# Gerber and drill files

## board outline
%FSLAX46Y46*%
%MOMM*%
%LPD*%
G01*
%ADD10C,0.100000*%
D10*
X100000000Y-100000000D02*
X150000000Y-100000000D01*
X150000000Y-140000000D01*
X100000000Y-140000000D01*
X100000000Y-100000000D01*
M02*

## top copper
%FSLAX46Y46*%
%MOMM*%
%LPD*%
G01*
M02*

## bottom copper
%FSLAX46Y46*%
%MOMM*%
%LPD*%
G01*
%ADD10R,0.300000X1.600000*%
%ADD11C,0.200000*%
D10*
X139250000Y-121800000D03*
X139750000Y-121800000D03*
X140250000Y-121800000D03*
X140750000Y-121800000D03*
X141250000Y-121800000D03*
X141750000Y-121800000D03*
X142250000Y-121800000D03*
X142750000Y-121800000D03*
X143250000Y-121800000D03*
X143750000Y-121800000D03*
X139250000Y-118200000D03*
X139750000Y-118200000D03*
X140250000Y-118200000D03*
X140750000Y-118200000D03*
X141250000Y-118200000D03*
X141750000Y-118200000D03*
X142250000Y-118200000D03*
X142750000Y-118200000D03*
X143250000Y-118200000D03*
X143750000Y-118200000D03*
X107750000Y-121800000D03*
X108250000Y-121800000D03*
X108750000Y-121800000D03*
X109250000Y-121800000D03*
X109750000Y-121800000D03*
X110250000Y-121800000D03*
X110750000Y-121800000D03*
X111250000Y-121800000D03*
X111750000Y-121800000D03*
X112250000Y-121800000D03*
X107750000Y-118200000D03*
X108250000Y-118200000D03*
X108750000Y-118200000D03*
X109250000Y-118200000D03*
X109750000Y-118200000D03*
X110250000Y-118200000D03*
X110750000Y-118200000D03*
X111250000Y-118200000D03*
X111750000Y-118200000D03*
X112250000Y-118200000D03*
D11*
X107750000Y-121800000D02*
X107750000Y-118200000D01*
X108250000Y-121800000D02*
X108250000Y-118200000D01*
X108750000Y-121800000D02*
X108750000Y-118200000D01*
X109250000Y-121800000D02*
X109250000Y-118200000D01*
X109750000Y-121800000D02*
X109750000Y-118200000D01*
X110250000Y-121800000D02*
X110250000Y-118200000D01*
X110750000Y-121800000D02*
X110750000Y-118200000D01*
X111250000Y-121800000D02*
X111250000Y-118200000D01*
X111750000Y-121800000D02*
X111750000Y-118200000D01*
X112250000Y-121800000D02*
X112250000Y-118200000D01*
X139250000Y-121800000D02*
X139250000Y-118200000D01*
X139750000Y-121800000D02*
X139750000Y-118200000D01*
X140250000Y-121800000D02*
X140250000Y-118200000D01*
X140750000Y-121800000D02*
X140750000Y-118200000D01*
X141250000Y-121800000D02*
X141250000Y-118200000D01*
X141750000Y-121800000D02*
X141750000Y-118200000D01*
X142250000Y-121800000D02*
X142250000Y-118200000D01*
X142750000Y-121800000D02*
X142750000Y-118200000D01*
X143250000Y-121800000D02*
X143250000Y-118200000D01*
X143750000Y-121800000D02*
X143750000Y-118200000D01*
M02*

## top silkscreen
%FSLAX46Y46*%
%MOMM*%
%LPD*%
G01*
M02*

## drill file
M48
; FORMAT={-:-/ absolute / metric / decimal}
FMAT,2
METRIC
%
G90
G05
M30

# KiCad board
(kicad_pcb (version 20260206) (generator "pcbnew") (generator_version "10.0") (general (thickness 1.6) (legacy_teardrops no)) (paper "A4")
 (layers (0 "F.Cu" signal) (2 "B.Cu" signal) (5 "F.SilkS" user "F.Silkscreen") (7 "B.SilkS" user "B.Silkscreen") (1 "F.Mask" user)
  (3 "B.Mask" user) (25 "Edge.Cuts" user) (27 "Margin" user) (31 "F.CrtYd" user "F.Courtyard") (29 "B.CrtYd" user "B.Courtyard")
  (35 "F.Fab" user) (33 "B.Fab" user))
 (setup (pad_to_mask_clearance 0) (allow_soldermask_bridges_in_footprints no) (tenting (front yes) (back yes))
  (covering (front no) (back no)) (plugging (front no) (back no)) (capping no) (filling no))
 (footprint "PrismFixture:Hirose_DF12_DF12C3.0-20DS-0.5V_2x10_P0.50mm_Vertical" (layer "B.Cu") (at 141.5 120)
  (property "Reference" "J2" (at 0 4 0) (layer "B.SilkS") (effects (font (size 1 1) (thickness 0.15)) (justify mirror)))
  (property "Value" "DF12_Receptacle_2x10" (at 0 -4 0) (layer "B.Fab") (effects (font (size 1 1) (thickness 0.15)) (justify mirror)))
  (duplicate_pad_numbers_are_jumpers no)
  (pad "" smd rect (at -2.25 -2) (size 0.28 1.2) (layers "B.Paste"))
  (pad "" smd rect (at -2.25 2) (size 0.28 1.2) (layers "B.Paste"))
  (pad "" smd rect (at -1.75 -2) (size 0.28 1.2) (layers "B.Paste"))
  (pad "" smd rect (at -1.75 2) (size 0.28 1.2) (layers "B.Paste"))
  (pad "" smd rect (at -1.25 -2) (size 0.28 1.2) (layers "B.Paste"))
  (pad "" smd rect (at -1.25 2) (size 0.28 1.2) (layers "B.Paste"))
  (pad "" smd rect (at -0.75 -2) (size 0.28 1.2) (layers "B.Paste"))
  (pad "" smd rect (at -0.75 2) (size 0.28 1.2) (layers "B.Paste"))
  (pad "" smd rect (at -0.25 -2) (size 0.28 1.2) (layers "B.Paste"))
  (pad "" smd rect (at -0.25 2) (size 0.28 1.2) (layers "B.Paste"))
  (pad "" smd rect (at 0.25 -2) (size 0.28 1.2) (layers "B.Paste"))
  (pad "" smd rect (at 0.25 2) (size 0.28 1.2) (layers "B.Paste"))
  (pad "" smd rect (at 0.75 -2) (size 0.28 1.2) (layers "B.Paste"))
  (pad "" smd rect (at 0.75 2) (size 0.28 1.2) (layers "B.Paste"))
  (pad "" smd rect (at 1.25 -2) (size 0.28 1.2) (layers "B.Paste"))
  (pad "" smd rect (at 1.25 2) (size 0.28 1.2) (layers "B.Paste"))
  (pad "" smd rect (at 1.75 -2) (size 0.28 1.2) (layers "B.Paste"))
  (pad "" smd rect (at 1.75 2) (size 0.28 1.2) (layers "B.Paste"))
  (pad "" smd rect (at 2.25 -2) (size 0.28 1.2) (layers "B.Paste"))
  (pad "" smd rect (at 2.25 2) (size 0.28 1.2) (layers "B.Paste"))
  (pad "1" smd rect (at -2.25 1.8) (size 0.3 1.6) (layers "B.Cu" "B.Mask") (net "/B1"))
  (pad "2" smd rect (at -1.75 1.8) (size 0.3 1.6) (layers "B.Cu" "B.Mask") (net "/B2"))
  (pad "3" smd rect (at -1.25 1.8) (size 0.3 1.6) (layers "B.Cu" "B.Mask") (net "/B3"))
  (pad "4" smd rect (at -0.75 1.8) (size 0.3 1.6) (layers "B.Cu" "B.Mask") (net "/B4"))
  (pad "5" smd rect (at -0.25 1.8) (size 0.3 1.6) (layers "B.Cu" "B.Mask") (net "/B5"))
  (pad "6" smd rect (at 0.25 1.8) (size 0.3 1.6) (layers "B.Cu" "B.Mask") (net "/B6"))
  (pad "7" smd rect (at 0.75 1.8) (size 0.3 1.6) (layers "B.Cu" "B.Mask") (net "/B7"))
  (pad "8" smd rect (at 1.25 1.8) (size 0.3 1.6) (layers "B.Cu" "B.Mask") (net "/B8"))
  (pad "9" smd rect (at 1.75 1.8) (size 0.3 1.6) (layers "B.Cu" "B.Mask") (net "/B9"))
  (pad "10" smd rect (at 2.25 1.8) (size 0.3 1.6) (layers "B.Cu" "B.Mask") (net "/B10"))
  (pad "11" smd rect (at -2.25 -1.8) (size 0.3 1.6) (layers "B.Cu" "B.Mask") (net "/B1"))
  (pad "12" smd rect (at -1.75 -1.8) (size 0.3 1.6) (layers "B.Cu" "B.Mask") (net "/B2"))
  (pad "13" smd rect (at -1.25 -1.8) (size 0.3 1.6) (layers "B.Cu" "B.Mask") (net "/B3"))
  (pad "14" smd rect (at -0.75 -1.8) (size 0.3 1.6) (layers "B.Cu" "B.Mask") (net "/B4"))
  (pad "15" smd rect (at -0.25 -1.8) (size 0.3 1.6) (layers "B.Cu" "B.Mask") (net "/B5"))
  (pad "16" smd rect (at 0.25 -1.8) (size 0.3 1.6) (layers "B.Cu" "B.Mask") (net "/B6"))
  (pad "17" smd rect (at 0.75 -1.8) (size 0.3 1.6) (layers "B.Cu" "B.Mask") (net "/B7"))
  (pad "18" smd rect (at 1.25 -1.8) (size 0.3 1.6) (layers "B.Cu" "B.Mask") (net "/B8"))
  (pad "19" smd rect (at 1.75 -1.8) (size 0.3 1.6) (layers "B.Cu" "B.Mask") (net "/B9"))
  (pad "20" smd rect (at 2.25 -1.8) (size 0.3 1.6) (layers "B.Cu" "B.Mask") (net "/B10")))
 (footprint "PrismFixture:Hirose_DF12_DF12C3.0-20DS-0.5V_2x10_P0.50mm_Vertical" (layer "B.Cu") (at 110 120)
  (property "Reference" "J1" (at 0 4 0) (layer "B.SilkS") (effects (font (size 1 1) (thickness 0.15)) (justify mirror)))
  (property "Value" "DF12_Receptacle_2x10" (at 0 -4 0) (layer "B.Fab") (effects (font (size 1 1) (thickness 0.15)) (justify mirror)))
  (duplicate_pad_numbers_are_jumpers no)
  (pad "" smd rect (at -2.25 -2) (size 0.28 1.2) (layers "B.Paste"))
  (pad "" smd rect (at -2.25 2) (size 0.28 1.2) (layers "B.Paste"))
  (pad "" smd rect (at -1.75 -2) (size 0.28 1.2) (layers "B.Paste"))
  (pad "" smd rect (at -1.75 2) (size 0.28 1.2) (layers "B.Paste"))
  (pad "" smd rect (at -1.25 -2) (size 0.28 1.2) (layers "B.Paste"))
  (pad "" smd rect (at -1.25 2) (size 0.28 1.2) (layers "B.Paste"))
  (pad "" smd rect (at -0.75 -2) (size 0.28 1.2) (layers "B.Paste"))
  (pad "" smd rect (at -0.75 2) (size 0.28 1.2) (layers "B.Paste"))
  (pad "" smd rect (at -0.25 -2) (size 0.28 1.2) (layers "B.Paste"))
  (pad "" smd rect (at -0.25 2) (size 0.28 1.2) (layers "B.Paste"))
  (pad "" smd rect (at 0.25 -2) (size 0.28 1.2) (layers "B.Paste"))
  (pad "" smd rect (at 0.25 2) (size 0.28 1.2) (layers "B.Paste"))
  (pad "" smd rect (at 0.75 -2) (size 0.28 1.2) (layers "B.Paste"))
  (pad "" smd rect (at 0.75 2) (size 0.28 1.2) (layers "B.Paste"))
  (pad "" smd rect (at 1.25 -2) (size 0.28 1.2) (layers "B.Paste"))
  (pad "" smd rect (at 1.25 2) (size 0.28 1.2) (layers "B.Paste"))
  (pad "" smd rect (at 1.75 -2) (size 0.28 1.2) (layers "B.Paste"))
  (pad "" smd rect (at 1.75 2) (size 0.28 1.2) (layers "B.Paste"))
  (pad "" smd rect (at 2.25 -2) (size 0.28 1.2) (layers "B.Paste"))
  (pad "" smd rect (at 2.25 2) (size 0.28 1.2) (layers "B.Paste"))
  (pad "1" smd rect (at -2.25 1.8) (size 0.3 1.6) (layers "B.Cu" "B.Mask") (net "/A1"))
  (pad "2" smd rect (at -1.75 1.8) (size 0.3 1.6) (layers "B.Cu" "B.Mask") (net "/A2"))
  (pad "3" smd rect (at -1.25 1.8) (size 0.3 1.6) (layers "B.Cu" "B.Mask") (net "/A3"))
  (pad "4" smd rect (at -0.75 1.8) (size 0.3 1.6) (layers "B.Cu" "B.Mask") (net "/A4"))
  (pad "5" smd rect (at -0.25 1.8) (size 0.3 1.6) (layers "B.Cu" "B.Mask") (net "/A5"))
  (pad "6" smd rect (at 0.25 1.8) (size 0.3 1.6) (layers "B.Cu" "B.Mask") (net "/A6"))
  (pad "7" smd rect (at 0.75 1.8) (size 0.3 1.6) (layers "B.Cu" "B.Mask") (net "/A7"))
  (pad "8" smd rect (at 1.25 1.8) (size 0.3 1.6) (layers "B.Cu" "B.Mask") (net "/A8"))
  (pad "9" smd rect (at 1.75 1.8) (size 0.3 1.6) (layers "B.Cu" "B.Mask") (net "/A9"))
  (pad "10" smd rect (at 2.25 1.8) (size 0.3 1.6) (layers "B.Cu" "B.Mask") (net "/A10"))
  (pad "11" smd rect (at -2.25 -1.8) (size 0.3 1.6) (layers "B.Cu" "B.Mask") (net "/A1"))
  (pad "12" smd rect (at -1.75 -1.8) (size 0.3 1.6) (layers "B.Cu" "B.Mask") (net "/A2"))
  (pad "13" smd rect (at -1.25 -1.8) (size 0.3 1.6) (layers "B.Cu" "B.Mask") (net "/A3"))
  (pad "14" smd rect (at -0.75 -1.8) (size 0.3 1.6) (layers "B.Cu" "B.Mask") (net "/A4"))
  (pad "15" smd rect (at -0.25 -1.8) (size 0.3 1.6) (layers "B.Cu" "B.Mask") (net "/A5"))
  (pad "16" smd rect (at 0.25 -1.8) (size 0.3 1.6) (layers "B.Cu" "B.Mask") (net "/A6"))
  (pad "17" smd rect (at 0.75 -1.8) (size 0.3 1.6) (layers "B.Cu" "B.Mask") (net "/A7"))
  (pad "18" smd rect (at 1.25 -1.8) (size 0.3 1.6) (layers "B.Cu" "B.Mask") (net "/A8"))
  (pad "19" smd rect (at 1.75 -1.8) (size 0.3 1.6) (layers "B.Cu" "B.Mask") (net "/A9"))
  (pad "20" smd rect (at 2.25 -1.8) (size 0.3 1.6) (layers "B.Cu" "B.Mask") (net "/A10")))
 (gr_rect (start 100 100) (end 150 140) (stroke (width 0.1) (type solid)) (fill no) (layer "Edge.Cuts"))
 (segment (start 107.75 121.8) (end 107.75 118.2) (width 0.2) (layer "B.Cu") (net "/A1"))
 (segment (start 108.25 121.8) (end 108.25 118.2) (width 0.2) (layer "B.Cu") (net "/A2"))
 (segment (start 108.75 121.8) (end 108.75 118.2) (width 0.2) (layer "B.Cu") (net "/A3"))
 (segment (start 109.25 121.8) (end 109.25 118.2) (width 0.2) (layer "B.Cu") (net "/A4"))
 (segment (start 109.75 121.8) (end 109.75 118.2) (width 0.2) (layer "B.Cu") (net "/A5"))
 (segment (start 110.25 121.8) (end 110.25 118.2) (width 0.2) (layer "B.Cu") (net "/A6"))
 (segment (start 110.75 121.8) (end 110.75 118.2) (width 0.2) (layer "B.Cu") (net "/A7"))
 (segment (start 111.25 121.8) (end 111.25 118.2) (width 0.2) (layer "B.Cu") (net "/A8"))
 (segment (start 111.75 121.8) (end 111.75 118.2) (width 0.2) (layer "B.Cu") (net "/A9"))
 (segment (start 112.25 121.8) (end 112.25 118.2) (width 0.2) (layer "B.Cu") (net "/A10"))
 (segment (start 139.25 121.8) (end 139.25 118.2) (width 0.2) (layer "B.Cu") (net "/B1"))
 (segment (start 139.75 121.8) (end 139.75 118.2) (width 0.2) (layer "B.Cu") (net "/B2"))
 (segment (start 140.25 121.8) (end 140.25 118.2) (width 0.2) (layer "B.Cu") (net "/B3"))
 (segment (start 140.75 121.8) (end 140.75 118.2) (width 0.2) (layer "B.Cu") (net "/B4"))
 (segment (start 141.25 121.8) (end 141.25 118.2) (width 0.2) (layer "B.Cu") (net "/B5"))
 (segment (start 141.75 121.8) (end 141.75 118.2) (width 0.2) (layer "B.Cu") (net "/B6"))
 (segment (start 142.25 121.8) (end 142.25 118.2) (width 0.2) (layer "B.Cu") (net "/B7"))
 (segment (start 142.75 121.8) (end 142.75 118.2) (width 0.2) (layer "B.Cu") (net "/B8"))
 (segment (start 143.25 121.8) (end 143.25 118.2) (width 0.2) (layer "B.Cu") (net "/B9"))
 (segment (start 143.75 121.8) (end 143.75 118.2) (width 0.2) (layer "B.Cu") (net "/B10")))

